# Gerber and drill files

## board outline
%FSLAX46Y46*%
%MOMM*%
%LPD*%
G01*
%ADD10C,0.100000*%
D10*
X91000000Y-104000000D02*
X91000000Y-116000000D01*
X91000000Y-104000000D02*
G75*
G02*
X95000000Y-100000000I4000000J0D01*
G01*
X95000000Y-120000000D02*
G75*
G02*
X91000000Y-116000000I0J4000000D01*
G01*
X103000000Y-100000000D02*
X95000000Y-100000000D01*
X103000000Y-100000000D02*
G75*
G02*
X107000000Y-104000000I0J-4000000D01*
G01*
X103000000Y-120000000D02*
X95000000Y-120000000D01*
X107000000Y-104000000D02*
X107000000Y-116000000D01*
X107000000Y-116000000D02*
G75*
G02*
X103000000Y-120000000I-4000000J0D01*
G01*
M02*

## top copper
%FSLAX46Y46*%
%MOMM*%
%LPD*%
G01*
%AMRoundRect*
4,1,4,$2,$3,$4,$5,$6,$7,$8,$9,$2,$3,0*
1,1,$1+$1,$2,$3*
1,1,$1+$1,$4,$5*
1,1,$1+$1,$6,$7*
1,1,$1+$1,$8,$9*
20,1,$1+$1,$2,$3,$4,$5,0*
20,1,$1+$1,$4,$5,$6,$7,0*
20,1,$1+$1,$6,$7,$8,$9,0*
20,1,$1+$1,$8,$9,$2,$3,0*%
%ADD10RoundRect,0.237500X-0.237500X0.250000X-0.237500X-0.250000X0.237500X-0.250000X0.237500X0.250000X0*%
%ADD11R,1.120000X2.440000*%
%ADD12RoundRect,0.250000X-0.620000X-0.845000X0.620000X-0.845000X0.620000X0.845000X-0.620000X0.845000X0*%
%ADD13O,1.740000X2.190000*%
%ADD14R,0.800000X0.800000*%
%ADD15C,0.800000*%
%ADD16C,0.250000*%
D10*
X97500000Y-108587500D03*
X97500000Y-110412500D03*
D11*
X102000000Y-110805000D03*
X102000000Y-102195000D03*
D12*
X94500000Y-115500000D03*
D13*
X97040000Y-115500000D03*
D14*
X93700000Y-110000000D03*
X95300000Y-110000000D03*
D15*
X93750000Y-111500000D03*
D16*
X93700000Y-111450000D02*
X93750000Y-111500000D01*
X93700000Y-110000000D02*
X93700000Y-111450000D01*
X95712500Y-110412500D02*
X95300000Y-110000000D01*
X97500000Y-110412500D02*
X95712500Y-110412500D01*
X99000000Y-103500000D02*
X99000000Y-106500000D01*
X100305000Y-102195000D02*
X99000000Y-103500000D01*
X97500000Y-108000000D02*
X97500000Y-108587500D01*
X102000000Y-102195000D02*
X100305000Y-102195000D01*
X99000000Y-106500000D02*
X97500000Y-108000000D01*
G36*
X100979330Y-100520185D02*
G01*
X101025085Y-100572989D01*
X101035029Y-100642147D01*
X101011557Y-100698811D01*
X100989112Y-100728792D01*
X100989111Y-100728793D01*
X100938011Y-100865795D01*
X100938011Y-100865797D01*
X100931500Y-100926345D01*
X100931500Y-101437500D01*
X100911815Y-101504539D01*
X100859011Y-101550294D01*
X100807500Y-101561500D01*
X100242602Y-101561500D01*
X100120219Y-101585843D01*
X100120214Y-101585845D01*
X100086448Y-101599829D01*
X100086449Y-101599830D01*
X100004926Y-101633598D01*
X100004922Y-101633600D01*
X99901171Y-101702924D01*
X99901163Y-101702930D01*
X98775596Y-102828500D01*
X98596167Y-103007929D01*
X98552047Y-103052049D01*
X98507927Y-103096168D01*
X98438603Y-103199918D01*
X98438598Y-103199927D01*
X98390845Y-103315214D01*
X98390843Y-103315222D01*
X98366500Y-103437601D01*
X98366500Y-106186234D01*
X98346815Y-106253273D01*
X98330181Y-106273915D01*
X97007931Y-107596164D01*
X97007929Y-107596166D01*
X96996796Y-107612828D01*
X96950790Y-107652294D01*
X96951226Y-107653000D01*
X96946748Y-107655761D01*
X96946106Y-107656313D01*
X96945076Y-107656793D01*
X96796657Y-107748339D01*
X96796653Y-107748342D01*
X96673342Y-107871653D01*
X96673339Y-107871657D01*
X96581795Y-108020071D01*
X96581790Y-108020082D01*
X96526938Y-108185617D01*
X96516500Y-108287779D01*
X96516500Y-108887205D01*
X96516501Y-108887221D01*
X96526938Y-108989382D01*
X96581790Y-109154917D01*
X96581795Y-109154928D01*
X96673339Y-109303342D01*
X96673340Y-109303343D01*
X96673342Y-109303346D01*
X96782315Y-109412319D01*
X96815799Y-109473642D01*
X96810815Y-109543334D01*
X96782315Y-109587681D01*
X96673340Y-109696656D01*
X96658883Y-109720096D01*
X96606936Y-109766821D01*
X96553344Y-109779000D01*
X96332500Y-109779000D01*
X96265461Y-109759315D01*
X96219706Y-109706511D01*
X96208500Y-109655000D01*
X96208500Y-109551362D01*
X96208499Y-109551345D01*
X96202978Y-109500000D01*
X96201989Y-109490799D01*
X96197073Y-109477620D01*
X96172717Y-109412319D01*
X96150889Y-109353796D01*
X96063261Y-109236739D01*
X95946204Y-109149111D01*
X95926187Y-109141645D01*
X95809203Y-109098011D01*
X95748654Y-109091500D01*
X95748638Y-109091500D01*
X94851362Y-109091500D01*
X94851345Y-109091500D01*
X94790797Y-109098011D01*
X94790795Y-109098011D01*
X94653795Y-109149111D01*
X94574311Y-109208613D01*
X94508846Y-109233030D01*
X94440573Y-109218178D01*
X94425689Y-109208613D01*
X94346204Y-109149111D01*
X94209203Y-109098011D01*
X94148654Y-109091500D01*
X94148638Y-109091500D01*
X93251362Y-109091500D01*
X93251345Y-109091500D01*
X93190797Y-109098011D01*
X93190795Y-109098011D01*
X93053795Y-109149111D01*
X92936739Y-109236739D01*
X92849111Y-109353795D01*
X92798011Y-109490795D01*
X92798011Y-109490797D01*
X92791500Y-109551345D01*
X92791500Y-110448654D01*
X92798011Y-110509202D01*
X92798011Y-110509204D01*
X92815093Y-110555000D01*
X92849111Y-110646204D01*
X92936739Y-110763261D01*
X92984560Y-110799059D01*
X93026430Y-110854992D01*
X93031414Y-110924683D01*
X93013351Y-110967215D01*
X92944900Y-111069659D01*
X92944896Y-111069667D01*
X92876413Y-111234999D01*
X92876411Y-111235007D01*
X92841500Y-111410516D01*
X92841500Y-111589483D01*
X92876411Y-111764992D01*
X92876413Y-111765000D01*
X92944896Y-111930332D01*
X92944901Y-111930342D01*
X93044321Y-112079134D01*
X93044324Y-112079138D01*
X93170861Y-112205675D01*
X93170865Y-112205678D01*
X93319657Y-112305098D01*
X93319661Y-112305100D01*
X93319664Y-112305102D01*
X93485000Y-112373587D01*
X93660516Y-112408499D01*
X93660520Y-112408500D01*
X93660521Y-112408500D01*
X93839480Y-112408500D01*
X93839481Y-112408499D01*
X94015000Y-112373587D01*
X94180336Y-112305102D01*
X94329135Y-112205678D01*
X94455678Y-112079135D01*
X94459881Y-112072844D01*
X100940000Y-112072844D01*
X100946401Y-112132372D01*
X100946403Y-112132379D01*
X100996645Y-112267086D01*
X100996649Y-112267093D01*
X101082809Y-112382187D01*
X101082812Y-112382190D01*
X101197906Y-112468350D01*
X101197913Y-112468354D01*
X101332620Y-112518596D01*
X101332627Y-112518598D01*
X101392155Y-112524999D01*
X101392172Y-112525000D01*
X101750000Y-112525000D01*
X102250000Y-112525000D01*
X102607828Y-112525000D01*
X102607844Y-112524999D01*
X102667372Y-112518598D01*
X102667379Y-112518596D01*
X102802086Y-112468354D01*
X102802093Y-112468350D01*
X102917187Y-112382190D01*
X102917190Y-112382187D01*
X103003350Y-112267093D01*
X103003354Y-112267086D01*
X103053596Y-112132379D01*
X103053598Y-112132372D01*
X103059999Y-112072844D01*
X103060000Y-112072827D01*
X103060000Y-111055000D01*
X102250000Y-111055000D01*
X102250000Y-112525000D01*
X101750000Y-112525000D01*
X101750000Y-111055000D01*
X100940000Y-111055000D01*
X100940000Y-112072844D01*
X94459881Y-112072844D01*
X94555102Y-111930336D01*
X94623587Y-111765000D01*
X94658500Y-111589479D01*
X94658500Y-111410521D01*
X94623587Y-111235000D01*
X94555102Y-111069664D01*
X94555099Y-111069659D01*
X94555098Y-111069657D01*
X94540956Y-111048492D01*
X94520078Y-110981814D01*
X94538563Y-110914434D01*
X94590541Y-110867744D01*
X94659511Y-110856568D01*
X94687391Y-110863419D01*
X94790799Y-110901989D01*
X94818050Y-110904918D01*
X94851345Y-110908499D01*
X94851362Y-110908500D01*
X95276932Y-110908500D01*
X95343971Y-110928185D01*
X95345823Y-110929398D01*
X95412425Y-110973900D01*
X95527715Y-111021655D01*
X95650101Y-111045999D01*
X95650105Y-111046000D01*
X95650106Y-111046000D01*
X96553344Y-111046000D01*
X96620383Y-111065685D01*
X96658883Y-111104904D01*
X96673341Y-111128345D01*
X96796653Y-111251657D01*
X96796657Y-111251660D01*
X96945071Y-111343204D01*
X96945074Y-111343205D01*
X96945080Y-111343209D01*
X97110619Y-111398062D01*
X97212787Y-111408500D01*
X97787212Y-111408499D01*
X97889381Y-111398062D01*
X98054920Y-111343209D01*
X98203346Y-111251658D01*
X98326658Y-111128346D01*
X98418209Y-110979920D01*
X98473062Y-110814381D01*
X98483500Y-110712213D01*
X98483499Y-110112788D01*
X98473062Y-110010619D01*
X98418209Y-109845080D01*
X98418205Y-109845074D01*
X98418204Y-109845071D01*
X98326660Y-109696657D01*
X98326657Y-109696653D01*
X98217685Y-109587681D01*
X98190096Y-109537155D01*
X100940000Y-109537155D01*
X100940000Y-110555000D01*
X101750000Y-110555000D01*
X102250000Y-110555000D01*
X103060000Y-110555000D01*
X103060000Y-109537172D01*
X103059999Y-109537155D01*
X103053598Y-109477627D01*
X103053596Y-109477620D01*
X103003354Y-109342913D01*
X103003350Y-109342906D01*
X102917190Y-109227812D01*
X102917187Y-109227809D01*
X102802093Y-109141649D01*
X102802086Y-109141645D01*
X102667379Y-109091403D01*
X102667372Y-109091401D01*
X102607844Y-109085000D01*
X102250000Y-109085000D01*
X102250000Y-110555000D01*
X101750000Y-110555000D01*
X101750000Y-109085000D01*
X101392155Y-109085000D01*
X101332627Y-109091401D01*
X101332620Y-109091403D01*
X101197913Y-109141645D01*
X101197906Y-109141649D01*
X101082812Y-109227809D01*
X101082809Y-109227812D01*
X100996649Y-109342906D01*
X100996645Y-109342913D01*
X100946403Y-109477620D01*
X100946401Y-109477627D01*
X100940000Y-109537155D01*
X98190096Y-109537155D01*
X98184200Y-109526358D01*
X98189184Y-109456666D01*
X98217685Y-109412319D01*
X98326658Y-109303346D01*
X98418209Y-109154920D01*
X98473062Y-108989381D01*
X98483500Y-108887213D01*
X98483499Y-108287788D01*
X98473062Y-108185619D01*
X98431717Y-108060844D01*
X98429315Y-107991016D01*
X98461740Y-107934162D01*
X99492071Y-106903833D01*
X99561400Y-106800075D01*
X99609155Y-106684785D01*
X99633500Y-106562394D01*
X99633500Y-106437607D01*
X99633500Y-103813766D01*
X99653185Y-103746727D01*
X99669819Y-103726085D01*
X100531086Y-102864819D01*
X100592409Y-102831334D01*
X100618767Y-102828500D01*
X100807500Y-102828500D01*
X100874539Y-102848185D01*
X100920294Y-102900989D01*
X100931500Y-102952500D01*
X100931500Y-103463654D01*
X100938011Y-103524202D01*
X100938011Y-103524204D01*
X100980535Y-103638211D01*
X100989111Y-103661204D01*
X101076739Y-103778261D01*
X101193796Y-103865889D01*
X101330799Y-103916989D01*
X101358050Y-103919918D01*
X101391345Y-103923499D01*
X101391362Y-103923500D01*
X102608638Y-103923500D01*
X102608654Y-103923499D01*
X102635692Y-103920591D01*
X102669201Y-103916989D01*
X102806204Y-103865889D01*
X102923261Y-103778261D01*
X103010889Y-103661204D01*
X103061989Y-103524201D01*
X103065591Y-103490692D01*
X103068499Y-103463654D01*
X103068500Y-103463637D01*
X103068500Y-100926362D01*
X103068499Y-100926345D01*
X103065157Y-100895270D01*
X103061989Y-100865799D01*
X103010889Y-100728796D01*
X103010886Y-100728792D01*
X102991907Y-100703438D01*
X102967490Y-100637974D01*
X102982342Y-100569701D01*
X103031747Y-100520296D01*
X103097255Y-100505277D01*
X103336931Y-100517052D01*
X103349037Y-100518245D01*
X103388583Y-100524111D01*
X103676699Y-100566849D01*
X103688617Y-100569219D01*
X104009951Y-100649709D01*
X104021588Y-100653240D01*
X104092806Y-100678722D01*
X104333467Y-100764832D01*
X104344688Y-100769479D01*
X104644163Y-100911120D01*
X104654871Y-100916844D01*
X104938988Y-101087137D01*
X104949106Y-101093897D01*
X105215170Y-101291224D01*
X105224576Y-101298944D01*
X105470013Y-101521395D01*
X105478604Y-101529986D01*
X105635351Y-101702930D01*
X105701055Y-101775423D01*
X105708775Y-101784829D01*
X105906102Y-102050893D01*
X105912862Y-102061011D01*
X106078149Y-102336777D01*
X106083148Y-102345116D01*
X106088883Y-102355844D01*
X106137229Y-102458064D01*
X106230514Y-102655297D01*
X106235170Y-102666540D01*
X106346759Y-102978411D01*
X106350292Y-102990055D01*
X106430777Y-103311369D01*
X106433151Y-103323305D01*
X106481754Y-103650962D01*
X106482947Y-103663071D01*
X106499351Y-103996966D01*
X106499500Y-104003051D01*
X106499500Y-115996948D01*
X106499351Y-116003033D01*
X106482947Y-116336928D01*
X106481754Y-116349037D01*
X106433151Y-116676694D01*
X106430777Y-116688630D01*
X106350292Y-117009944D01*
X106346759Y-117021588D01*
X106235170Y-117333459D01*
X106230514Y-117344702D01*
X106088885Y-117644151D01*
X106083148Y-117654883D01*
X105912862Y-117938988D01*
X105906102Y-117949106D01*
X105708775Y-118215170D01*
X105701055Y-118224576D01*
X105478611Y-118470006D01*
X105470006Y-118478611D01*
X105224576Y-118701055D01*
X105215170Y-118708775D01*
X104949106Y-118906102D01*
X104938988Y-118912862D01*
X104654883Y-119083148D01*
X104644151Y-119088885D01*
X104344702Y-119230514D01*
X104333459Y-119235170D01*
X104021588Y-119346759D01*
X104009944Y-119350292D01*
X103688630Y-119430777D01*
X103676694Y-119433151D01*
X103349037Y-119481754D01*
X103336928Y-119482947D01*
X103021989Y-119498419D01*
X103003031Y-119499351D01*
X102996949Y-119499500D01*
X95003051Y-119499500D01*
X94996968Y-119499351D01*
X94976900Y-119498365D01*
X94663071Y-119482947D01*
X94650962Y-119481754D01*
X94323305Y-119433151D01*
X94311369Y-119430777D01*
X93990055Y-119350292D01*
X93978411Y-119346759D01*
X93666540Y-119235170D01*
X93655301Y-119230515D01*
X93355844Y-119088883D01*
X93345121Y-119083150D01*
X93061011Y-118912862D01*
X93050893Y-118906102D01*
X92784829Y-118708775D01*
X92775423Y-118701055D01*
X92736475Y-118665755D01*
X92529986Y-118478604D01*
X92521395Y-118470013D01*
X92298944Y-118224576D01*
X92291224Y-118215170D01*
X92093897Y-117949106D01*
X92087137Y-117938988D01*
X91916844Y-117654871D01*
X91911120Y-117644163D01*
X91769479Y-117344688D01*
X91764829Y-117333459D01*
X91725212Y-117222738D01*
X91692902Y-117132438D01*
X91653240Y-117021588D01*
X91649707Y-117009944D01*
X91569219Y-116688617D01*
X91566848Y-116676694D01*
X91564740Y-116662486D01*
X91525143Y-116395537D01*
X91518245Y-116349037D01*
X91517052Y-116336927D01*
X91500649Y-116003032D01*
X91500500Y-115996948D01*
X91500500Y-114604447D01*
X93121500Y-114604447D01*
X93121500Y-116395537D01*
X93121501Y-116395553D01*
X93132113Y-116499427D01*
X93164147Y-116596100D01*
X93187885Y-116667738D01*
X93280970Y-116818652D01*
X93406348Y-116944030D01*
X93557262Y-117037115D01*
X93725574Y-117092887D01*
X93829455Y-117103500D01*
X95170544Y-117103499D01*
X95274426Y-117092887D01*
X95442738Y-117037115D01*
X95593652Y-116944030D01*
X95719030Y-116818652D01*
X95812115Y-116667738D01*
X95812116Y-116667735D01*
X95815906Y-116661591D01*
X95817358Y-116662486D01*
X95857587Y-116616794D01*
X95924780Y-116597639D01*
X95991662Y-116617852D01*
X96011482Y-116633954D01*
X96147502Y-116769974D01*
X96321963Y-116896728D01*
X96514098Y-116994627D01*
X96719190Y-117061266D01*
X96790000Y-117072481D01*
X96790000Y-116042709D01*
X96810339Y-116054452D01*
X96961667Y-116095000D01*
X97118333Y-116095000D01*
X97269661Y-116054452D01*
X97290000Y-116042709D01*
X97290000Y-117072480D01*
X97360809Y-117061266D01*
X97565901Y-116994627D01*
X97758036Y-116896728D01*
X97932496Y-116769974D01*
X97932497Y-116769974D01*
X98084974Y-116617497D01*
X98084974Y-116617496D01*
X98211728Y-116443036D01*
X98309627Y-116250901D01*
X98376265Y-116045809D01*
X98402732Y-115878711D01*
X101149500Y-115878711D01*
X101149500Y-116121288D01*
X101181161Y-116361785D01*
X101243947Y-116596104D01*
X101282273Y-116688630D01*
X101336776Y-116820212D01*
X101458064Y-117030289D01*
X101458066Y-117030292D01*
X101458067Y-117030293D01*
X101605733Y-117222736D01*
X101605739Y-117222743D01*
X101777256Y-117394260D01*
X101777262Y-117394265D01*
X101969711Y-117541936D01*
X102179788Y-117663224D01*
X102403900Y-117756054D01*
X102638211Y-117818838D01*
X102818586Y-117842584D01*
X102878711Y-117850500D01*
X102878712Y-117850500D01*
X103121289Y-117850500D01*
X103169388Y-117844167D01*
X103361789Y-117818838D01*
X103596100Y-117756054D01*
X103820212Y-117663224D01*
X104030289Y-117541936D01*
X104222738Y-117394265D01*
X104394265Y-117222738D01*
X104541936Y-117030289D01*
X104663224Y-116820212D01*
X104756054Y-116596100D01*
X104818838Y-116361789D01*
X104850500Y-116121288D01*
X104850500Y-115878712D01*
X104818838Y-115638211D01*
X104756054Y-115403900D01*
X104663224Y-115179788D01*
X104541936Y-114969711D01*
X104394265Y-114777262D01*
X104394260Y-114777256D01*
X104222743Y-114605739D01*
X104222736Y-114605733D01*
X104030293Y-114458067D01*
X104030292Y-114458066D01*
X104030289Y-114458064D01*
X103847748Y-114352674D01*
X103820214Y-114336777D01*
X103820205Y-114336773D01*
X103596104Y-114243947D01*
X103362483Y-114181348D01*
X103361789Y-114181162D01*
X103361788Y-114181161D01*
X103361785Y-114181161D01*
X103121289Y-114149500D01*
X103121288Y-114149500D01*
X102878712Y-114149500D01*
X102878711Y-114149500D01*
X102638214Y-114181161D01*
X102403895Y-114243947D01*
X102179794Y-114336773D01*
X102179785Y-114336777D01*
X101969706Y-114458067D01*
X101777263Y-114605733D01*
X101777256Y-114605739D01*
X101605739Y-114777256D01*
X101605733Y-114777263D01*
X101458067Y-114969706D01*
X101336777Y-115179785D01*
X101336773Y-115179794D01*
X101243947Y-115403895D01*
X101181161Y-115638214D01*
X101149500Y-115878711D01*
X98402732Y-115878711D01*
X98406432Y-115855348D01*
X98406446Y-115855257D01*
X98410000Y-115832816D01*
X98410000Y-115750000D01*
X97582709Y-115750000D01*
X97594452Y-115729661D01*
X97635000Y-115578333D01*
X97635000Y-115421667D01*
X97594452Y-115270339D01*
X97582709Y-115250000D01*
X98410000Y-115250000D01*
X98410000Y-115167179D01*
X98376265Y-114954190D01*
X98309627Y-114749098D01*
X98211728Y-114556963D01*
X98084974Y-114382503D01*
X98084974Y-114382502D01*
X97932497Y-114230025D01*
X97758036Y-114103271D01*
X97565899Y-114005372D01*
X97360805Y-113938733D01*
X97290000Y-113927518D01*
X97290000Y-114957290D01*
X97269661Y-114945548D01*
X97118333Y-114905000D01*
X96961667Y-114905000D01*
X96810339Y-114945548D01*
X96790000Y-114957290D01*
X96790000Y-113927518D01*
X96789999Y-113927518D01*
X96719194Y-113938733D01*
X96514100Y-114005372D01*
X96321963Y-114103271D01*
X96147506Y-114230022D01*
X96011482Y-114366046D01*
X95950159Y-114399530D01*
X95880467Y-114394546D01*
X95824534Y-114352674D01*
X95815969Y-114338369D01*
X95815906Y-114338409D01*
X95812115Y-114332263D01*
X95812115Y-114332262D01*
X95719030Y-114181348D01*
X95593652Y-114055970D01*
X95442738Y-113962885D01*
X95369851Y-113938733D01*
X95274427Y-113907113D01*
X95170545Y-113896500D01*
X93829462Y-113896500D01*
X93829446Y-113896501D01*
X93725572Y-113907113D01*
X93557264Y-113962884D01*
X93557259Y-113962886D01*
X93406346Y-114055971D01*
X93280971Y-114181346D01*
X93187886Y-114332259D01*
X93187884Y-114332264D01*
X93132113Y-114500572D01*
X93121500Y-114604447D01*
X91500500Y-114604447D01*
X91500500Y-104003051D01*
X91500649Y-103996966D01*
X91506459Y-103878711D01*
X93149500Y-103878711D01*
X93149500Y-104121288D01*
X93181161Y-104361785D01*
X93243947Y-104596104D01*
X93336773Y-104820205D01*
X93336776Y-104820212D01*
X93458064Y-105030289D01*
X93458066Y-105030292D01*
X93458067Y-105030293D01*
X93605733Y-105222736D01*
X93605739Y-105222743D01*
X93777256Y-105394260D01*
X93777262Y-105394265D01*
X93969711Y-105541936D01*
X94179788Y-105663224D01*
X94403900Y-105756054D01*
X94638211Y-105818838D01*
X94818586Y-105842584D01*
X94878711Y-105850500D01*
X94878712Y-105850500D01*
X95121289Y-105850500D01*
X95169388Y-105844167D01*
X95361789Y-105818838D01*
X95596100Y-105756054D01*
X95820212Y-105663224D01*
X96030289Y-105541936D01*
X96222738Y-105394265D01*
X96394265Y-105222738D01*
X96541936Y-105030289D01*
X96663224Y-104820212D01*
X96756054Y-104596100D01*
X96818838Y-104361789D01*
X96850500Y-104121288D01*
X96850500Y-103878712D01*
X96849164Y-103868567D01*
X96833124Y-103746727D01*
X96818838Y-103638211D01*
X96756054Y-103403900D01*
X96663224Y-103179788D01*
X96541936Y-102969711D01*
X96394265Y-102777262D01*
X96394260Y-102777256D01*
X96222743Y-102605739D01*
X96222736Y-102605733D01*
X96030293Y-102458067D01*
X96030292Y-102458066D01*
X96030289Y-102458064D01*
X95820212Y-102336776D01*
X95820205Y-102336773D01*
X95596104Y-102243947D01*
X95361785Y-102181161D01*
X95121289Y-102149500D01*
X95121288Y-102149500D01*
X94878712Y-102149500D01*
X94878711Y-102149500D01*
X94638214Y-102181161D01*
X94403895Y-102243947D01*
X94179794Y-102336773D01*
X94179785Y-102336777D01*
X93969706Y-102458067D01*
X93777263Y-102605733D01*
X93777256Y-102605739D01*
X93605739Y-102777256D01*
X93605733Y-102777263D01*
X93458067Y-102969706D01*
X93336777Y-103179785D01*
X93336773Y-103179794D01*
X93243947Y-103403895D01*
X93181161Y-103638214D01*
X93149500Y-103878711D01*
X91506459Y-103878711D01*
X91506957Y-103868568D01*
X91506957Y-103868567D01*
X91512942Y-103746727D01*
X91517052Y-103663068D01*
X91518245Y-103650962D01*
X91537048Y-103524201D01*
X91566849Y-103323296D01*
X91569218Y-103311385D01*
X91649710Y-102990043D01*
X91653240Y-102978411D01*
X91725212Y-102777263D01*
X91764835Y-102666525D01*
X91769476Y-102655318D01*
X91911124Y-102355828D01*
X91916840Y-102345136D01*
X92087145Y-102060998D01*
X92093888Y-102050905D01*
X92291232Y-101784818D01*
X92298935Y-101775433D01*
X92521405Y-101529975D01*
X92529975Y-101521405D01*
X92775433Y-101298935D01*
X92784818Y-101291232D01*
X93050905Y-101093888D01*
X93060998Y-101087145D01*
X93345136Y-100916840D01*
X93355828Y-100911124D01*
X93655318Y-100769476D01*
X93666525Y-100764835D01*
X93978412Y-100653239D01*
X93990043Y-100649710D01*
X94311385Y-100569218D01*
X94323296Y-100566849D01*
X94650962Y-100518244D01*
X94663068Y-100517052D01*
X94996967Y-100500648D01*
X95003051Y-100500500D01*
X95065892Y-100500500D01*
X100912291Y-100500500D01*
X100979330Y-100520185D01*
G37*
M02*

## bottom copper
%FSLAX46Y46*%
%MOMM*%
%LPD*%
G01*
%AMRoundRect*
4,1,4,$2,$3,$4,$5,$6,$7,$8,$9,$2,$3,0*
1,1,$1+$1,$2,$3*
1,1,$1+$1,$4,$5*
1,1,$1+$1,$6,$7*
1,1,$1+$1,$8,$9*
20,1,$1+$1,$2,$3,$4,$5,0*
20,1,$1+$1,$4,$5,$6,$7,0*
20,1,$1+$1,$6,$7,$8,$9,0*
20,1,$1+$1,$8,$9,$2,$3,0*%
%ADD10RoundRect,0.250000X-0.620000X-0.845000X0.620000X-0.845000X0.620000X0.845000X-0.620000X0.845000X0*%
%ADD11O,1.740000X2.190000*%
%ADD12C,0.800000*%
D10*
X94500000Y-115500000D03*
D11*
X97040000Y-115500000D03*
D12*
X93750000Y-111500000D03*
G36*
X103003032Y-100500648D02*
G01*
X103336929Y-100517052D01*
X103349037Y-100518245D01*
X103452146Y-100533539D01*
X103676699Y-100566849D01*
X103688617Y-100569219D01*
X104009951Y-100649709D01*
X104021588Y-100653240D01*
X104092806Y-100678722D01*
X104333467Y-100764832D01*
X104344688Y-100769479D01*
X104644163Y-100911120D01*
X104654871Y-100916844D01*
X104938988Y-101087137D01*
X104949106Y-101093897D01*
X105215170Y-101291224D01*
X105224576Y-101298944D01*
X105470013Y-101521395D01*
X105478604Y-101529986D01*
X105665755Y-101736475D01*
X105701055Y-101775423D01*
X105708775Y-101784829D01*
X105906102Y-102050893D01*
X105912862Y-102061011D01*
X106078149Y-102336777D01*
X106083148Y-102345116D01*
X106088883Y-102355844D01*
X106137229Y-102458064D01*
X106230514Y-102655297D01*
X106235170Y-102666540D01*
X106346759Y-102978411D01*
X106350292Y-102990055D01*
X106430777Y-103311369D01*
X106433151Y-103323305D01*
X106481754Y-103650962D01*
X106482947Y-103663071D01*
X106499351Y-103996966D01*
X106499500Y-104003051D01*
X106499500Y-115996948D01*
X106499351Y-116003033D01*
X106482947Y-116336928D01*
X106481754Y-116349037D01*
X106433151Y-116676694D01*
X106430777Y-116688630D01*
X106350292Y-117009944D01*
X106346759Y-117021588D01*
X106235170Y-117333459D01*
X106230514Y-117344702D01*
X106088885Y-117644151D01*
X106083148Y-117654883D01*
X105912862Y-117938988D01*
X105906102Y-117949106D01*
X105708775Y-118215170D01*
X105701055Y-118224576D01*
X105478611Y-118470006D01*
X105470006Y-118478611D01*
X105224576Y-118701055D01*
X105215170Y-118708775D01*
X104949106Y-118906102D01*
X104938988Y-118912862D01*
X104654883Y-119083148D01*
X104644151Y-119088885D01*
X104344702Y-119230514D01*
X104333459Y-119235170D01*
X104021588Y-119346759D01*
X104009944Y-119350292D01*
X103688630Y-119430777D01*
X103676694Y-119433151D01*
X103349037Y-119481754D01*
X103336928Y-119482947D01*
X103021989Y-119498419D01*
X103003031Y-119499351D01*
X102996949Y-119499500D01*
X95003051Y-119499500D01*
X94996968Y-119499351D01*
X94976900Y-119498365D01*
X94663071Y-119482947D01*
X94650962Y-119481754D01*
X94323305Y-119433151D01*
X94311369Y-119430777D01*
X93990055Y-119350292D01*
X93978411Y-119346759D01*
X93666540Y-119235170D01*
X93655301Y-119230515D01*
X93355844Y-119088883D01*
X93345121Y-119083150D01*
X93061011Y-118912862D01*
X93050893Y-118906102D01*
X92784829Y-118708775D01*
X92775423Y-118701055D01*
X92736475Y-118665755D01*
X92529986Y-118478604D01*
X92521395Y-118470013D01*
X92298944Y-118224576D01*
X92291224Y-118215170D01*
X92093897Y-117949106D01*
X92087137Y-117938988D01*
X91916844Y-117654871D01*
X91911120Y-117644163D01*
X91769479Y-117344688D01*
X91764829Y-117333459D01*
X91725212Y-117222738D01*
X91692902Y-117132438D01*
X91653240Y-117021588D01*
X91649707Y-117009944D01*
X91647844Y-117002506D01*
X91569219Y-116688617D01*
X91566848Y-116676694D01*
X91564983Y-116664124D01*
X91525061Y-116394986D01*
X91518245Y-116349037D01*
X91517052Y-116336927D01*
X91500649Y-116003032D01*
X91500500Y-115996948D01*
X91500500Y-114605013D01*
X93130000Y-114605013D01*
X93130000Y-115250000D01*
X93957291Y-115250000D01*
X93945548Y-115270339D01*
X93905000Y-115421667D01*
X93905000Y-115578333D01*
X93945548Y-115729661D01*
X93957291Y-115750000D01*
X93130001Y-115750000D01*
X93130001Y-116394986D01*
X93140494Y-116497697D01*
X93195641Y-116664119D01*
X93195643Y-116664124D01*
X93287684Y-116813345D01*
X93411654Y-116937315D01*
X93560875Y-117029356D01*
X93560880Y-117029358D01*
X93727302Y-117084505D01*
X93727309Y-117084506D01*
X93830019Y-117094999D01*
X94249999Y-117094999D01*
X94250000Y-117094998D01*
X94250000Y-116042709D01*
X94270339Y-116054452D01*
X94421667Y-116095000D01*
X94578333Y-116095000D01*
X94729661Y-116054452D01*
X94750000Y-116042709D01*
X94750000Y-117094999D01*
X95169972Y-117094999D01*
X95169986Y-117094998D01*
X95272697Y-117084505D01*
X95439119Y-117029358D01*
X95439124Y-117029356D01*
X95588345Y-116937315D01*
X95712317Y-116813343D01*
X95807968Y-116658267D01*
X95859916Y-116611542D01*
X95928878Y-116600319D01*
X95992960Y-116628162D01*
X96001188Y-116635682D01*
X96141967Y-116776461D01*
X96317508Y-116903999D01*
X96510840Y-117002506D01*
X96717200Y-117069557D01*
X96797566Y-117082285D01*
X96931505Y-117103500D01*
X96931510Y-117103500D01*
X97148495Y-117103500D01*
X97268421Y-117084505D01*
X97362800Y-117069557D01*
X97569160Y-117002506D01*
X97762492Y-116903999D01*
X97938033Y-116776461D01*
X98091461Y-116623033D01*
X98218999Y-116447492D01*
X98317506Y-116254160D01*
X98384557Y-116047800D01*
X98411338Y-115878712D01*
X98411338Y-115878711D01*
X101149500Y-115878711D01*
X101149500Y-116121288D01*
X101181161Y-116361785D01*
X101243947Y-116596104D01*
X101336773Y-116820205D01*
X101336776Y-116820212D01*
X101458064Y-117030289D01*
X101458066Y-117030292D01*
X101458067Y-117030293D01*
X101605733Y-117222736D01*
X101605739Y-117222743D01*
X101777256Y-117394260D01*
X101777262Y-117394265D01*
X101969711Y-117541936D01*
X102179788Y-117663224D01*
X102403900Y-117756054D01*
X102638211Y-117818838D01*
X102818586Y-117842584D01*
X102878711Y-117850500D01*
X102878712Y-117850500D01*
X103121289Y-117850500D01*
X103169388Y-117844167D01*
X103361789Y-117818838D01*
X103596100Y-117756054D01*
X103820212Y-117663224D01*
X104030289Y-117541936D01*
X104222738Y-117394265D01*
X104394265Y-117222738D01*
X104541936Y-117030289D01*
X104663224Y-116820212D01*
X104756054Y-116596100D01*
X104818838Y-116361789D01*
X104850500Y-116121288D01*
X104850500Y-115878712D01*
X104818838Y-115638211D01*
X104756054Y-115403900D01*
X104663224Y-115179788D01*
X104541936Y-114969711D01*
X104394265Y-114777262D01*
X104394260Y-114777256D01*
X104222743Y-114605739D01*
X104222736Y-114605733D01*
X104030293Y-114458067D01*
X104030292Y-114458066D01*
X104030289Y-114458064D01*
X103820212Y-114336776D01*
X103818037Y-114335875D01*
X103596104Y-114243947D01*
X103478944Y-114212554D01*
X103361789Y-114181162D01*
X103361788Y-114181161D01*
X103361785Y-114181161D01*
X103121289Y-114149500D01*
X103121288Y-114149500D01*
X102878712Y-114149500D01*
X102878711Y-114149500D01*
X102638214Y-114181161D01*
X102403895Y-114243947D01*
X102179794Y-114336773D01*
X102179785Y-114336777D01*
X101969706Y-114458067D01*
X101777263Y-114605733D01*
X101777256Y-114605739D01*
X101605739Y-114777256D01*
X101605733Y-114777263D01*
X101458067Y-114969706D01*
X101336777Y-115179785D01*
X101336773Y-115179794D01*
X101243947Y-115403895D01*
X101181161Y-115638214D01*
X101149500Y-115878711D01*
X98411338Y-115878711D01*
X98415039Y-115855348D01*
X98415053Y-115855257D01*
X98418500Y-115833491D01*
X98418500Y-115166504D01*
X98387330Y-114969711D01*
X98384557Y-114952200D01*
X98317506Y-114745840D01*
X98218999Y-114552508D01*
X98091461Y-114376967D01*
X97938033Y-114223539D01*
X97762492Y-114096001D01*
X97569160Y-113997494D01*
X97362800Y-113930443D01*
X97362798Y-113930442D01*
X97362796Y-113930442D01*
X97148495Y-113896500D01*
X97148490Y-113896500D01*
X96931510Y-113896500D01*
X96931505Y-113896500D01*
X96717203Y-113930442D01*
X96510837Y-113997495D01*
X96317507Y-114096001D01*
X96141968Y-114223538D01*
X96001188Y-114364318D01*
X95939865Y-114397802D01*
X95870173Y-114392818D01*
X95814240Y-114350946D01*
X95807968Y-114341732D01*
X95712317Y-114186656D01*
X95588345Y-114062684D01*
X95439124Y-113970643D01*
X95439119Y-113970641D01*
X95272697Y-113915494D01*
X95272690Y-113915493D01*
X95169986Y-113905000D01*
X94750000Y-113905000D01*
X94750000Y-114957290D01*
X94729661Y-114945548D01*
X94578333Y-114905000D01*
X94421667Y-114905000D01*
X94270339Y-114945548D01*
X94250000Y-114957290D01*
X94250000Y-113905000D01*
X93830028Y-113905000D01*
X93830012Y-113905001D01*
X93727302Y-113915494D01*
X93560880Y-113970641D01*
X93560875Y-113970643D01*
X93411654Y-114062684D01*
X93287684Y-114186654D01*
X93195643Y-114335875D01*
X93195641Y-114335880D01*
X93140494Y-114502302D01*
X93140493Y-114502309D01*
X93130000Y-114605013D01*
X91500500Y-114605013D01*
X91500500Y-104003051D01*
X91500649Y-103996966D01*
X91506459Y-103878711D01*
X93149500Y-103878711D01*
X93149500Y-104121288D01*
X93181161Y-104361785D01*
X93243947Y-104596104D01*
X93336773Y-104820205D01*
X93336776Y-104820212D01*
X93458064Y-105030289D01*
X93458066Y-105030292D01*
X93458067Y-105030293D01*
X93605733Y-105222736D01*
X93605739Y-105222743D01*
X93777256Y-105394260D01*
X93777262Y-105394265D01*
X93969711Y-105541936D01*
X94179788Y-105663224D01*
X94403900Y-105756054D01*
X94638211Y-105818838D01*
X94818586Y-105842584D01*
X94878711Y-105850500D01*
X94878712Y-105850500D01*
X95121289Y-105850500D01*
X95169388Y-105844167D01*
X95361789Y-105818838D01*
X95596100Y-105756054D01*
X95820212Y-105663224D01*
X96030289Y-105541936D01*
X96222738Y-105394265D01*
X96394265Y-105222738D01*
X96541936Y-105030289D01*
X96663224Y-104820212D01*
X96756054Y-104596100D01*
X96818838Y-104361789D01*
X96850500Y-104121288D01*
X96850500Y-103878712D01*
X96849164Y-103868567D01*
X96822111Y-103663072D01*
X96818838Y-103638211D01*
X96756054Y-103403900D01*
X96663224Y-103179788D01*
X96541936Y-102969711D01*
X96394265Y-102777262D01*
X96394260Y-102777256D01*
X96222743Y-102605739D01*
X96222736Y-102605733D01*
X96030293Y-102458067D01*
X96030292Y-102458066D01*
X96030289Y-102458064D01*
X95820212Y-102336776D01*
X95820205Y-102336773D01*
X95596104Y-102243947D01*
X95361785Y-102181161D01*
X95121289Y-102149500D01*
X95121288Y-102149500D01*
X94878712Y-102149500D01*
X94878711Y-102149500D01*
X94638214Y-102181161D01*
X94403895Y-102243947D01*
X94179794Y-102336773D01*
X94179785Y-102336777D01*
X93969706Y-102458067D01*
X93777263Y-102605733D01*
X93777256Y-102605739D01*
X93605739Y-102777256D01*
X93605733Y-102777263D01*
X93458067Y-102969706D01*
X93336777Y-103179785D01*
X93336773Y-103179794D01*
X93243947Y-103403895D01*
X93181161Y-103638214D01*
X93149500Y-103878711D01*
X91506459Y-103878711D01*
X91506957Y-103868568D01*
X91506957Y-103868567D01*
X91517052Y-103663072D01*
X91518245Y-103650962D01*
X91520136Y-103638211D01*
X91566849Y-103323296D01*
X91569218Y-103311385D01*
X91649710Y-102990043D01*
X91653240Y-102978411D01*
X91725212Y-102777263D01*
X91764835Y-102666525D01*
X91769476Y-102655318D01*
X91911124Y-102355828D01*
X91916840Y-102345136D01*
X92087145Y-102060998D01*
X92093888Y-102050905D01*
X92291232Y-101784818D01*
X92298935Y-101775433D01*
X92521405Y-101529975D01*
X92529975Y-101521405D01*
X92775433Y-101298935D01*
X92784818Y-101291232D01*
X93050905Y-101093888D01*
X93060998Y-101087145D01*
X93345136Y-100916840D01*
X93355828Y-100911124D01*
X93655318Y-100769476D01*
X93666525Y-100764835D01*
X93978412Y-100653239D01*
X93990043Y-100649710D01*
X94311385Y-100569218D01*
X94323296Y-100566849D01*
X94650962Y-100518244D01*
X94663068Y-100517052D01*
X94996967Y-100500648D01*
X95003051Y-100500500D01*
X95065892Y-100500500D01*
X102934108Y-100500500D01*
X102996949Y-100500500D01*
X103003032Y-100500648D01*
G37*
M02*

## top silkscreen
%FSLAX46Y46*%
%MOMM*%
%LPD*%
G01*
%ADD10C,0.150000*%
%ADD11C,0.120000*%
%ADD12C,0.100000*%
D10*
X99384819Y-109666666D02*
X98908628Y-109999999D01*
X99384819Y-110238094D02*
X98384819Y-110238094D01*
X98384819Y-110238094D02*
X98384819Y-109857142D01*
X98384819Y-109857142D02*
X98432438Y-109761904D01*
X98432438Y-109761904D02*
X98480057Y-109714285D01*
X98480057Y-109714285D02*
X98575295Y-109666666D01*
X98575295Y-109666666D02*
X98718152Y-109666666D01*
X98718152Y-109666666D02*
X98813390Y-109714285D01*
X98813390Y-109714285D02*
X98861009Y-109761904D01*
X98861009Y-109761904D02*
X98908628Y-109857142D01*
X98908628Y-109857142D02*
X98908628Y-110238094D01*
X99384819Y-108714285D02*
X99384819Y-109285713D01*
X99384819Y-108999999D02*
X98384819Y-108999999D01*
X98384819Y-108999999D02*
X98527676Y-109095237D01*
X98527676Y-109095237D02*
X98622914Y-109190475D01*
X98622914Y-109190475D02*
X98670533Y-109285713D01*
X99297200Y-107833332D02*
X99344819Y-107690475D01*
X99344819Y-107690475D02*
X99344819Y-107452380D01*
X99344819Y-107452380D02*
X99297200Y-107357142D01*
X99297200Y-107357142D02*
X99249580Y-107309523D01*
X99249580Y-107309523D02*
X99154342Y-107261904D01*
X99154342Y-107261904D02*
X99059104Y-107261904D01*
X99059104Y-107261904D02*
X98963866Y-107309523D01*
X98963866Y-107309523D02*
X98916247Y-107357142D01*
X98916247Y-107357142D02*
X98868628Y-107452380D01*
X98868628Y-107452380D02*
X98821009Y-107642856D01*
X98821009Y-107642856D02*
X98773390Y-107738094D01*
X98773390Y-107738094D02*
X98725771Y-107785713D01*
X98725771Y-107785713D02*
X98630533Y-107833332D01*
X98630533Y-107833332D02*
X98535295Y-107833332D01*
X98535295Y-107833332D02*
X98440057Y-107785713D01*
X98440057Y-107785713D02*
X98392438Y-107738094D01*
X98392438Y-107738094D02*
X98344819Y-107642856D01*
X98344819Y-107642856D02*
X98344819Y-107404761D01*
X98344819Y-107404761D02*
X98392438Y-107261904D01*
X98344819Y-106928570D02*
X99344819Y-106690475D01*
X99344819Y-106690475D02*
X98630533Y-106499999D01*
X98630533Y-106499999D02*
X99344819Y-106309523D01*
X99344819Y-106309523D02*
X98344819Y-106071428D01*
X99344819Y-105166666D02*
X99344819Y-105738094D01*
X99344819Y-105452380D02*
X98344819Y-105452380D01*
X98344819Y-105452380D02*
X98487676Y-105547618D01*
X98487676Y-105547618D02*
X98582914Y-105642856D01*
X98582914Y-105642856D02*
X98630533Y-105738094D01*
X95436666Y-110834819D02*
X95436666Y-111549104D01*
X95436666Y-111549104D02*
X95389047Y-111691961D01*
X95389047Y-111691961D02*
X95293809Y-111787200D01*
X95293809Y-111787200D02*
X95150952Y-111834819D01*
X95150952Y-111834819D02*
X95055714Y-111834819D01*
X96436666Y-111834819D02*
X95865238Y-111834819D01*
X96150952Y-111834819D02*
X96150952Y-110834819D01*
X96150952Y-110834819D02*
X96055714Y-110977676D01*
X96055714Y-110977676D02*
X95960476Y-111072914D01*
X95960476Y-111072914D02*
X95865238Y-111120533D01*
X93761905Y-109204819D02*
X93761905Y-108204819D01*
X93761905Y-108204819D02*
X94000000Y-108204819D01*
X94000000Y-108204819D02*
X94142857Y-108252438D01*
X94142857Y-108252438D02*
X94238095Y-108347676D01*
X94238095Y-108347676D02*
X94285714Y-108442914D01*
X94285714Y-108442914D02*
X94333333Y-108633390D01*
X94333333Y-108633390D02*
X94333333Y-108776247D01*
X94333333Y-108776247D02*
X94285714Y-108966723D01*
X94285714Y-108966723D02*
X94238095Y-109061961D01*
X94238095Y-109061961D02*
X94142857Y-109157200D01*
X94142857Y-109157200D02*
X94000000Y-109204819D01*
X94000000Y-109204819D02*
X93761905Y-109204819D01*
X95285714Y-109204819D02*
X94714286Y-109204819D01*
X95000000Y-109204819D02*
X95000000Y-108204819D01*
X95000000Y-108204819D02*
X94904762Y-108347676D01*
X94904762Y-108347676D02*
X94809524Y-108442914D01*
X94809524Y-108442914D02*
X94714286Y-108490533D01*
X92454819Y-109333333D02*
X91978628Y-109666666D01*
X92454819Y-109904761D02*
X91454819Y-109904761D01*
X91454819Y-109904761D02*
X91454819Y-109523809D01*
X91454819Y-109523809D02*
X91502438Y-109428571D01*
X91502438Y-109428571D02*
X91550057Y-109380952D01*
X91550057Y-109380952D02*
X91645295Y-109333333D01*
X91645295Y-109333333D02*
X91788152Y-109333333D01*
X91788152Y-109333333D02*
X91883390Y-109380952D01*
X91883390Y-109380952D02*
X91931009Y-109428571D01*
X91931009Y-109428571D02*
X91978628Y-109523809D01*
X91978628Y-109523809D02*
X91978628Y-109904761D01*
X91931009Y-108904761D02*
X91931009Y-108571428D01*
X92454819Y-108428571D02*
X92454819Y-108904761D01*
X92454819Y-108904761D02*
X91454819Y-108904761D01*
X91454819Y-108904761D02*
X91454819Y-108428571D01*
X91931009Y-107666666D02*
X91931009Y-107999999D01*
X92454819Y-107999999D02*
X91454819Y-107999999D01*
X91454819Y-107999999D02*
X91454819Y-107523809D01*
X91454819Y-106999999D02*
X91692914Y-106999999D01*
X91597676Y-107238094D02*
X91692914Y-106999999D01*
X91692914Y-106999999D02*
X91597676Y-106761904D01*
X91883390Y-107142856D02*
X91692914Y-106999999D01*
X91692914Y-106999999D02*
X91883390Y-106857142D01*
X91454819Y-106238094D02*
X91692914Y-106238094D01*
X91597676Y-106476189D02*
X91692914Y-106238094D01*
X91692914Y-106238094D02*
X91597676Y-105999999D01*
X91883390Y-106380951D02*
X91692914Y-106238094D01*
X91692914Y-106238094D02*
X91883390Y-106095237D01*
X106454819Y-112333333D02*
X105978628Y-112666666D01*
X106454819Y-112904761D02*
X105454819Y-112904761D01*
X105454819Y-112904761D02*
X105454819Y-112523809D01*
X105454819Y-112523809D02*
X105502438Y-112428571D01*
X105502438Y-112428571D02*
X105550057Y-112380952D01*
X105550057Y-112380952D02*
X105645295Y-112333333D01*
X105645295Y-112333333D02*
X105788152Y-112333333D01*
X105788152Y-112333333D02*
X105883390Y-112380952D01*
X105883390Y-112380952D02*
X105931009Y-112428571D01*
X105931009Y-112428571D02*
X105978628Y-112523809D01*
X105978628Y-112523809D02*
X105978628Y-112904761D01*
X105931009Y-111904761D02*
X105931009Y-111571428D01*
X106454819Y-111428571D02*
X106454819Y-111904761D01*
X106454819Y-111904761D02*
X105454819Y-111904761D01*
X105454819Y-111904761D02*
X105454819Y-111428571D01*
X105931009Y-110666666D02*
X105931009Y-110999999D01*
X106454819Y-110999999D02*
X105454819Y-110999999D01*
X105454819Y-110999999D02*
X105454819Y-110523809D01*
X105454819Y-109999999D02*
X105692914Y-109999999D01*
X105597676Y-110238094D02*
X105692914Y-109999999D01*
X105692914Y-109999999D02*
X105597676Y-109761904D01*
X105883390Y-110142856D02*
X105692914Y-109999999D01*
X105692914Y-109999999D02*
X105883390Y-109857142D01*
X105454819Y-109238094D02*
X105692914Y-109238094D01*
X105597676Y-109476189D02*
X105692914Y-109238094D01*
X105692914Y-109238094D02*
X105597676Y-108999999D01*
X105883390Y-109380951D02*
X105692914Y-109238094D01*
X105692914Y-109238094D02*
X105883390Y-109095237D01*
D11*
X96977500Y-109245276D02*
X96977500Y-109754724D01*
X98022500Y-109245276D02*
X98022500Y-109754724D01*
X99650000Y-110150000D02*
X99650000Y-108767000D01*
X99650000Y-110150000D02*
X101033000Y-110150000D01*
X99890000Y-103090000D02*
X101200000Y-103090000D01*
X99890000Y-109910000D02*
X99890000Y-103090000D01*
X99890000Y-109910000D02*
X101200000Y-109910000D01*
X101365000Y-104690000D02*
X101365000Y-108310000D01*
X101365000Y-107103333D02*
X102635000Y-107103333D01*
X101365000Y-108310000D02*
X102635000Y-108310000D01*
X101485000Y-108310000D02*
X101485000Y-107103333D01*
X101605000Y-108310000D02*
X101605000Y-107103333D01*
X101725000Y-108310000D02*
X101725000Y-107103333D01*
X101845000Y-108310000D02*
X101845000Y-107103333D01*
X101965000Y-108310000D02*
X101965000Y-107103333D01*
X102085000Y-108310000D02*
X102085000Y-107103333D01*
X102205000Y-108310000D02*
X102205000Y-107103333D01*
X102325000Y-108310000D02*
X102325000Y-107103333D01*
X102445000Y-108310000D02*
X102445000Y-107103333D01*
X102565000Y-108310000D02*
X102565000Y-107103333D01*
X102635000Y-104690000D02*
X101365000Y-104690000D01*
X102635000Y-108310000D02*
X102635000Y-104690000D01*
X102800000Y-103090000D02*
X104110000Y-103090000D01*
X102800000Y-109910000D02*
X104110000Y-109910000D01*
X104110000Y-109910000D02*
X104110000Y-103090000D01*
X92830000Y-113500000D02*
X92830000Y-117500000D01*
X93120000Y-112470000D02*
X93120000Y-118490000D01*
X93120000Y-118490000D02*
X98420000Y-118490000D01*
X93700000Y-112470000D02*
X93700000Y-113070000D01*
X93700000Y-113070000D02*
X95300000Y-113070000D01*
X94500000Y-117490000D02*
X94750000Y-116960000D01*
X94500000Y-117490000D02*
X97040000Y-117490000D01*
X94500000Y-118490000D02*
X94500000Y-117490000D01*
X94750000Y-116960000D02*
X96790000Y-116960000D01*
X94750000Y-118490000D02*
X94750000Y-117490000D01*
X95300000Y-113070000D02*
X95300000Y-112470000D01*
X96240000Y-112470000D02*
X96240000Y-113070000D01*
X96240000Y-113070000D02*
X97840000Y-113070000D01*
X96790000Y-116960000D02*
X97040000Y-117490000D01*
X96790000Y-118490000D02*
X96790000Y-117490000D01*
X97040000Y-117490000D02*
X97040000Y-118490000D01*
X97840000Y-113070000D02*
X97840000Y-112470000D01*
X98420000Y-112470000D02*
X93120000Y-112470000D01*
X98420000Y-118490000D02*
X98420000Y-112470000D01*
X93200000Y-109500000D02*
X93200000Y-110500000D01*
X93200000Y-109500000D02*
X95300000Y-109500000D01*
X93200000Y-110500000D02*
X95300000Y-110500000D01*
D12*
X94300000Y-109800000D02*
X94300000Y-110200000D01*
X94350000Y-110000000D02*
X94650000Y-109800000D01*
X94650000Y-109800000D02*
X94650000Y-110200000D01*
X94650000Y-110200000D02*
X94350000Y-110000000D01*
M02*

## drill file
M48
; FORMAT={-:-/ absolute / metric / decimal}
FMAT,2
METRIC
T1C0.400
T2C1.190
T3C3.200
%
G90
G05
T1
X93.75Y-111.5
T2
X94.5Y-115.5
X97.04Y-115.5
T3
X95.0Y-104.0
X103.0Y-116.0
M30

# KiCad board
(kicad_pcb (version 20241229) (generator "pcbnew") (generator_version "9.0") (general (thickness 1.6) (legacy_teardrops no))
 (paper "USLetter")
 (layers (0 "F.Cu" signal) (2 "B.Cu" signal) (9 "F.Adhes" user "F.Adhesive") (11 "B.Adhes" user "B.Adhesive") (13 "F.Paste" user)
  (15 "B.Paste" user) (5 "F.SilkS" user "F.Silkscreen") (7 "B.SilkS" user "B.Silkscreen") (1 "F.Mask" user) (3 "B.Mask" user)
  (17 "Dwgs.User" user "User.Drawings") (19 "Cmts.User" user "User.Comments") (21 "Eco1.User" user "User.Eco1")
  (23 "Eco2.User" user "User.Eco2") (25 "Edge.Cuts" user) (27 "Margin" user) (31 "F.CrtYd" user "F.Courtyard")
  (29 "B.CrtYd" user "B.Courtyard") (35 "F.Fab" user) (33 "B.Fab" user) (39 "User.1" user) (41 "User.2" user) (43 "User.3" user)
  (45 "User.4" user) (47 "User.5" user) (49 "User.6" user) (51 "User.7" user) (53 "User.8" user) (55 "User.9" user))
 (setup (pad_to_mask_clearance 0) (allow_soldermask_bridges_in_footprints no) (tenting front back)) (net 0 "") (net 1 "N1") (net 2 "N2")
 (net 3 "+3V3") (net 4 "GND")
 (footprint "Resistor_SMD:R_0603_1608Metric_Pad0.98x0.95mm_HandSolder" (layer "F.Cu") (at 97.5 109.5 -90)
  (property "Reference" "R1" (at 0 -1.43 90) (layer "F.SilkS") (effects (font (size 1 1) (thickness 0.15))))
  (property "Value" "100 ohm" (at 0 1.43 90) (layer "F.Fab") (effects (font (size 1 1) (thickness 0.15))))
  (fp_line (start -0.254724 0.5225) (end 0.254724 0.5225) (stroke (width 0.12) (type solid)) (layer "F.SilkS"))
  (fp_line (start -0.254724 -0.5225) (end 0.254724 -0.5225) (stroke (width 0.12) (type solid)) (layer "F.SilkS"))
  (pad "1" smd roundrect (at -0.9125 0 270) (size 0.975 0.95) (layers "F.Cu" "F.Mask" "F.Paste") (roundrect_rratio 0.25) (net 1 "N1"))
  (pad "2" smd roundrect (at 0.9125 0 270) (size 0.975 0.95) (layers "F.Cu" "F.Mask" "F.Paste") (roundrect_rratio 0.25) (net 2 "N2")))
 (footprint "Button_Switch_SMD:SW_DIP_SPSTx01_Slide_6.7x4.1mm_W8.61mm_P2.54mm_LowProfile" (layer "F.Cu") (at 102 106.5 90)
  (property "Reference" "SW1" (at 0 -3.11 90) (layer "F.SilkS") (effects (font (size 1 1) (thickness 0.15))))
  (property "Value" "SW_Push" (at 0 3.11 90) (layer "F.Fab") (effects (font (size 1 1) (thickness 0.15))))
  (fp_line (start -3.65 -2.35) (end -2.267 -2.35) (stroke (width 0.12) (type solid)) (layer "F.SilkS"))
  (fp_line (start -3.65 -2.35) (end -3.65 -0.967) (stroke (width 0.12) (type solid)) (layer "F.SilkS"))
  (fp_line (start 3.41 -2.11) (end 3.41 -0.8) (stroke (width 0.12) (type solid)) (layer "F.SilkS"))
  (fp_line (start -3.41 -2.11) (end 3.41 -2.11) (stroke (width 0.12) (type solid)) (layer "F.SilkS"))
  (fp_line (start -3.41 -2.11) (end -3.41 -0.8) (stroke (width 0.12) (type solid)) (layer "F.SilkS"))
  (fp_line (start 1.81 -0.635) (end -1.81 -0.635) (stroke (width 0.12) (type solid)) (layer "F.SilkS"))
  (fp_line (start -0.603333 -0.635) (end -0.603333 0.635) (stroke (width 0.12) (type solid)) (layer "F.SilkS"))
  (fp_line (start -1.81 -0.635) (end -1.81 0.635) (stroke (width 0.12) (type solid)) (layer "F.SilkS"))
  (fp_line (start -1.81 -0.515) (end -0.603333 -0.515) (stroke (width 0.12) (type solid)) (layer "F.SilkS"))
  (fp_line (start -1.81 -0.395) (end -0.603333 -0.395) (stroke (width 0.12) (type solid)) (layer "F.SilkS"))
  (fp_line (start -1.81 -0.275) (end -0.603333 -0.275) (stroke (width 0.12) (type solid)) (layer "F.SilkS"))
  (fp_line (start -1.81 -0.155) (end -0.603333 -0.155) (stroke (width 0.12) (type solid)) (layer "F.SilkS"))
  (fp_line (start -1.81 -0.035) (end -0.603333 -0.035) (stroke (width 0.12) (type solid)) (layer "F.SilkS"))
  (fp_line (start -1.81 0.085) (end -0.603333 0.085) (stroke (width 0.12) (type solid)) (layer "F.SilkS"))
  (fp_line (start -1.81 0.205) (end -0.603333 0.205) (stroke (width 0.12) (type solid)) (layer "F.SilkS"))
  (fp_line (start -1.81 0.325) (end -0.603333 0.325) (stroke (width 0.12) (type solid)) (layer "F.SilkS"))
  (fp_line (start -1.81 0.445) (end -0.603333 0.445) (stroke (width 0.12) (type solid)) (layer "F.SilkS"))
  (fp_line (start -1.81 0.565) (end -0.603333 0.565) (stroke (width 0.12) (type solid)) (layer "F.SilkS"))
  (fp_line (start 1.81 0.635) (end 1.81 -0.635) (stroke (width 0.12) (type solid)) (layer "F.SilkS"))
  (fp_line (start -1.81 0.635) (end 1.81 0.635) (stroke (width 0.12) (type solid)) (layer "F.SilkS"))
  (fp_line (start 3.41 0.8) (end 3.41 2.11) (stroke (width 0.12) (type solid)) (layer "F.SilkS"))
  (fp_line (start -3.41 0.8) (end -3.41 2.11) (stroke (width 0.12) (type solid)) (layer "F.SilkS"))
  (fp_line (start -3.41 2.11) (end 3.41 2.11) (stroke (width 0.12) (type solid)) (layer "F.SilkS"))
  (pad "1" smd rect (at -4.305 0 90) (size 2.44 1.12) (layers "F.Cu" "F.Mask" "F.Paste") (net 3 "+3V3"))
  (pad "2" smd rect (at 4.305 0 90) (size 2.44 1.12) (layers "F.Cu" "F.Mask" "F.Paste") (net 1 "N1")))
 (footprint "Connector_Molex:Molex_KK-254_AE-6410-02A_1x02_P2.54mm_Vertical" (layer "F.Cu") (at 94.5 115.5)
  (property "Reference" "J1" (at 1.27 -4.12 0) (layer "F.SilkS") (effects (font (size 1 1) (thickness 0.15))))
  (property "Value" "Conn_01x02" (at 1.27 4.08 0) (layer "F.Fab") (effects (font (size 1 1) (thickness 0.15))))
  (fp_line (start -1.67 -2) (end -1.67 2) (stroke (width 0.12) (type solid)) (layer "F.SilkS"))
  (fp_line (start -1.38 -3.03) (end -1.38 2.99) (stroke (width 0.12) (type solid)) (layer "F.SilkS"))
  (fp_line (start -1.38 2.99) (end 3.92 2.99) (stroke (width 0.12) (type solid)) (layer "F.SilkS"))
  (fp_line (start -0.8 -3.03) (end -0.8 -2.43) (stroke (width 0.12) (type solid)) (layer "F.SilkS"))
  (fp_line (start -0.8 -2.43) (end 0.8 -2.43) (stroke (width 0.12) (type solid)) (layer "F.SilkS"))
  (fp_line (start 0 1.99) (end 0.25 1.46) (stroke (width 0.12) (type solid)) (layer "F.SilkS"))
  (fp_line (start 0 1.99) (end 2.54 1.99) (stroke (width 0.12) (type solid)) (layer "F.SilkS"))
  (fp_line (start 0 2.99) (end 0 1.99) (stroke (width 0.12) (type solid)) (layer "F.SilkS"))
  (fp_line (start 0.25 1.46) (end 2.29 1.46) (stroke (width 0.12) (type solid)) (layer "F.SilkS"))
  (fp_line (start 0.25 2.99) (end 0.25 1.99) (stroke (width 0.12) (type solid)) (layer "F.SilkS"))
  (fp_line (start 0.8 -2.43) (end 0.8 -3.03) (stroke (width 0.12) (type solid)) (layer "F.SilkS"))
  (fp_line (start 1.74 -3.03) (end 1.74 -2.43) (stroke (width 0.12) (type solid)) (layer "F.SilkS"))
  (fp_line (start 1.74 -2.43) (end 3.34 -2.43) (stroke (width 0.12) (type solid)) (layer "F.SilkS"))
  (fp_line (start 2.29 1.46) (end 2.54 1.99) (stroke (width 0.12) (type solid)) (layer "F.SilkS"))
  (fp_line (start 2.29 2.99) (end 2.29 1.99) (stroke (width 0.12) (type solid)) (layer "F.SilkS"))
  (fp_line (start 2.54 1.99) (end 2.54 2.99) (stroke (width 0.12) (type solid)) (layer "F.SilkS"))
  (fp_line (start 3.34 -2.43) (end 3.34 -3.03) (stroke (width 0.12) (type solid)) (layer "F.SilkS"))
  (fp_line (start 3.92 -3.03) (end -1.38 -3.03) (stroke (width 0.12) (type solid)) (layer "F.SilkS"))
  (fp_line (start 3.92 2.99) (end 3.92 -3.03) (stroke (width 0.12) (type solid)) (layer "F.SilkS"))
  (pad "1" thru_hole roundrect (at 0 0) (size 1.74 2.19) (drill 1.19) (layers "*.Cu" "*.Mask") (remove_unused_layers no)
   (roundrect_rratio 0.143678) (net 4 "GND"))
  (pad "2" thru_hole oval (at 2.54 0) (size 1.74 2.19) (drill 1.19) (layers "*.Cu" "*.Mask") (remove_unused_layers no) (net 3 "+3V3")))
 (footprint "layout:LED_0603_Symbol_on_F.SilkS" (layer "F.Cu") (at 94.5 110)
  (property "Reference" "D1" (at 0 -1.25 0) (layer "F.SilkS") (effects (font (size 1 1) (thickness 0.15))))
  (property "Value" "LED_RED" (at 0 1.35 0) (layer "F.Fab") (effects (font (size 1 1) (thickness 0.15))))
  (fp_line (start -1.3 -0.5) (end -1.3 0.5) (stroke (width 0.12) (type solid)) (layer "F.SilkS"))
  (fp_line (start -1.3 -0.5) (end 0.8 -0.5) (stroke (width 0.12) (type solid)) (layer "F.SilkS"))
  (fp_line (start -1.3 0.5) (end 0.8 0.5) (stroke (width 0.12) (type solid)) (layer "F.SilkS"))
  (fp_line (start -0.2 -0.2) (end -0.2 0.2) (stroke (width 0.1) (type solid)) (layer "F.SilkS"))
  (fp_line (start -0.15 0) (end 0.15 -0.2) (stroke (width 0.1) (type solid)) (layer "F.SilkS"))
  (fp_line (start 0.15 -0.2) (end 0.15 0.2) (stroke (width 0.1) (type solid)) (layer "F.SilkS"))
  (fp_line (start 0.15 0.2) (end -0.15 0) (stroke (width 0.1) (type solid)) (layer "F.SilkS"))
  (pad "1" smd rect (at -0.8 0 180) (size 0.8 0.8) (layers "F.Cu" "F.Mask" "F.Paste") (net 4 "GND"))
  (pad "2" smd rect (at 0.8 0 180) (size 0.8 0.8) (layers "F.Cu" "F.Mask" "F.Paste") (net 2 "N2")))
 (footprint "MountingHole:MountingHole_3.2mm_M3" (layer "F.Cu") (at 95 104)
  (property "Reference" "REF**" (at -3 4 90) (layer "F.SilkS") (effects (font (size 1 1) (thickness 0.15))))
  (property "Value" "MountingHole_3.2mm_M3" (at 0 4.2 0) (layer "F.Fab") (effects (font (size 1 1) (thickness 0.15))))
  (pad "" np_thru_hole circle (at 0 0) (size 3.2 3.2) (drill 3.2) (layers "*.Cu" "*.Mask")))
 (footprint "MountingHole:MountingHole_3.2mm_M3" (layer "F.Cu") (at 103 116)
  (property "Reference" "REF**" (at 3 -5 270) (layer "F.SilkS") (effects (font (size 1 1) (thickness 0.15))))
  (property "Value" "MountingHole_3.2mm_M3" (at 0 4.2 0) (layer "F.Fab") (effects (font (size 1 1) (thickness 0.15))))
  (pad "" np_thru_hole circle (at 0 0) (size 3.2 3.2) (drill 3.2) (layers "*.Cu" "*.Mask")))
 (gr_line (start 91 104) (end 91 116) (stroke (width 0.1) (type default)) (layer "Edge.Cuts"))
 (gr_arc (start 91 104) (mid 92.171573 101.171573) (end 95 100) (stroke (width 0.1) (type default)) (layer "Edge.Cuts"))
 (gr_arc (start 95 120) (mid 92.171573 118.828427) (end 91 116) (stroke (width 0.1) (type default)) (layer "Edge.Cuts"))
 (gr_line (start 103 100) (end 95 100) (stroke (width 0.1) (type default)) (layer "Edge.Cuts"))
 (gr_arc (start 103 100) (mid 105.828427 101.171573) (end 107 104) (stroke (width 0.1) (type default)) (layer "Edge.Cuts"))
 (gr_line (start 103 120) (end 95 120) (stroke (width 0.1) (type default)) (layer "Edge.Cuts"))
 (gr_line (start 107 104) (end 107 116) (stroke (width 0.1) (type default)) (layer "Edge.Cuts"))
 (gr_arc (start 107 116) (mid 105.828427 118.828427) (end 103 120) (stroke (width 0.1) (type default)) (layer "Edge.Cuts"))
 (segment (start 93.7 111.45) (end 93.75 111.5) (width 0.25) (layer "F.Cu") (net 4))
 (segment (start 93.7 110) (end 93.7 111.45) (width 0.25) (layer "F.Cu") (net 4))
 (via (at 93.75 111.5) (size 0.8) (drill 0.4) (layers "F.Cu" "B.Cu") (free yes) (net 4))
 (segment (start 95.7125 110.4125) (end 95.3 110) (width 0.25) (layer "F.Cu") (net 2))
 (segment (start 97.5 110.4125) (end 95.7125 110.4125) (width 0.25) (layer "F.Cu") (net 2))
 (segment (start 99 103.5) (end 99 106.5) (width 0.25) (layer "F.Cu") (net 1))
 (segment (start 100.305 102.195) (end 99 103.5) (width 0.25) (layer "F.Cu") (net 1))
 (segment (start 97.5 108) (end 97.5 108.5875) (width 0.25) (layer "F.Cu") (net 1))
 (segment (start 102 102.195) (end 100.305 102.195) (width 0.25) (layer "F.Cu") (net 1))
 (segment (start 99 106.5) (end 97.5 108) (width 0.25) (layer "F.Cu") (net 1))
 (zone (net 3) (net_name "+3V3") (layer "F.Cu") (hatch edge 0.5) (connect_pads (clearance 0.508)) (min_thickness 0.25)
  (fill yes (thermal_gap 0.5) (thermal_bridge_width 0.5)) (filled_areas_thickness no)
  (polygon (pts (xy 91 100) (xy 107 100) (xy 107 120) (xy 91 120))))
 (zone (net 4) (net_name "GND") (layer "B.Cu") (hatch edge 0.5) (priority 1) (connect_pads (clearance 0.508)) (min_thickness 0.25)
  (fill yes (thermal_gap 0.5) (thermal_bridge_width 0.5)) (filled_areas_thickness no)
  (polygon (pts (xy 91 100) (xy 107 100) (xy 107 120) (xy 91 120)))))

